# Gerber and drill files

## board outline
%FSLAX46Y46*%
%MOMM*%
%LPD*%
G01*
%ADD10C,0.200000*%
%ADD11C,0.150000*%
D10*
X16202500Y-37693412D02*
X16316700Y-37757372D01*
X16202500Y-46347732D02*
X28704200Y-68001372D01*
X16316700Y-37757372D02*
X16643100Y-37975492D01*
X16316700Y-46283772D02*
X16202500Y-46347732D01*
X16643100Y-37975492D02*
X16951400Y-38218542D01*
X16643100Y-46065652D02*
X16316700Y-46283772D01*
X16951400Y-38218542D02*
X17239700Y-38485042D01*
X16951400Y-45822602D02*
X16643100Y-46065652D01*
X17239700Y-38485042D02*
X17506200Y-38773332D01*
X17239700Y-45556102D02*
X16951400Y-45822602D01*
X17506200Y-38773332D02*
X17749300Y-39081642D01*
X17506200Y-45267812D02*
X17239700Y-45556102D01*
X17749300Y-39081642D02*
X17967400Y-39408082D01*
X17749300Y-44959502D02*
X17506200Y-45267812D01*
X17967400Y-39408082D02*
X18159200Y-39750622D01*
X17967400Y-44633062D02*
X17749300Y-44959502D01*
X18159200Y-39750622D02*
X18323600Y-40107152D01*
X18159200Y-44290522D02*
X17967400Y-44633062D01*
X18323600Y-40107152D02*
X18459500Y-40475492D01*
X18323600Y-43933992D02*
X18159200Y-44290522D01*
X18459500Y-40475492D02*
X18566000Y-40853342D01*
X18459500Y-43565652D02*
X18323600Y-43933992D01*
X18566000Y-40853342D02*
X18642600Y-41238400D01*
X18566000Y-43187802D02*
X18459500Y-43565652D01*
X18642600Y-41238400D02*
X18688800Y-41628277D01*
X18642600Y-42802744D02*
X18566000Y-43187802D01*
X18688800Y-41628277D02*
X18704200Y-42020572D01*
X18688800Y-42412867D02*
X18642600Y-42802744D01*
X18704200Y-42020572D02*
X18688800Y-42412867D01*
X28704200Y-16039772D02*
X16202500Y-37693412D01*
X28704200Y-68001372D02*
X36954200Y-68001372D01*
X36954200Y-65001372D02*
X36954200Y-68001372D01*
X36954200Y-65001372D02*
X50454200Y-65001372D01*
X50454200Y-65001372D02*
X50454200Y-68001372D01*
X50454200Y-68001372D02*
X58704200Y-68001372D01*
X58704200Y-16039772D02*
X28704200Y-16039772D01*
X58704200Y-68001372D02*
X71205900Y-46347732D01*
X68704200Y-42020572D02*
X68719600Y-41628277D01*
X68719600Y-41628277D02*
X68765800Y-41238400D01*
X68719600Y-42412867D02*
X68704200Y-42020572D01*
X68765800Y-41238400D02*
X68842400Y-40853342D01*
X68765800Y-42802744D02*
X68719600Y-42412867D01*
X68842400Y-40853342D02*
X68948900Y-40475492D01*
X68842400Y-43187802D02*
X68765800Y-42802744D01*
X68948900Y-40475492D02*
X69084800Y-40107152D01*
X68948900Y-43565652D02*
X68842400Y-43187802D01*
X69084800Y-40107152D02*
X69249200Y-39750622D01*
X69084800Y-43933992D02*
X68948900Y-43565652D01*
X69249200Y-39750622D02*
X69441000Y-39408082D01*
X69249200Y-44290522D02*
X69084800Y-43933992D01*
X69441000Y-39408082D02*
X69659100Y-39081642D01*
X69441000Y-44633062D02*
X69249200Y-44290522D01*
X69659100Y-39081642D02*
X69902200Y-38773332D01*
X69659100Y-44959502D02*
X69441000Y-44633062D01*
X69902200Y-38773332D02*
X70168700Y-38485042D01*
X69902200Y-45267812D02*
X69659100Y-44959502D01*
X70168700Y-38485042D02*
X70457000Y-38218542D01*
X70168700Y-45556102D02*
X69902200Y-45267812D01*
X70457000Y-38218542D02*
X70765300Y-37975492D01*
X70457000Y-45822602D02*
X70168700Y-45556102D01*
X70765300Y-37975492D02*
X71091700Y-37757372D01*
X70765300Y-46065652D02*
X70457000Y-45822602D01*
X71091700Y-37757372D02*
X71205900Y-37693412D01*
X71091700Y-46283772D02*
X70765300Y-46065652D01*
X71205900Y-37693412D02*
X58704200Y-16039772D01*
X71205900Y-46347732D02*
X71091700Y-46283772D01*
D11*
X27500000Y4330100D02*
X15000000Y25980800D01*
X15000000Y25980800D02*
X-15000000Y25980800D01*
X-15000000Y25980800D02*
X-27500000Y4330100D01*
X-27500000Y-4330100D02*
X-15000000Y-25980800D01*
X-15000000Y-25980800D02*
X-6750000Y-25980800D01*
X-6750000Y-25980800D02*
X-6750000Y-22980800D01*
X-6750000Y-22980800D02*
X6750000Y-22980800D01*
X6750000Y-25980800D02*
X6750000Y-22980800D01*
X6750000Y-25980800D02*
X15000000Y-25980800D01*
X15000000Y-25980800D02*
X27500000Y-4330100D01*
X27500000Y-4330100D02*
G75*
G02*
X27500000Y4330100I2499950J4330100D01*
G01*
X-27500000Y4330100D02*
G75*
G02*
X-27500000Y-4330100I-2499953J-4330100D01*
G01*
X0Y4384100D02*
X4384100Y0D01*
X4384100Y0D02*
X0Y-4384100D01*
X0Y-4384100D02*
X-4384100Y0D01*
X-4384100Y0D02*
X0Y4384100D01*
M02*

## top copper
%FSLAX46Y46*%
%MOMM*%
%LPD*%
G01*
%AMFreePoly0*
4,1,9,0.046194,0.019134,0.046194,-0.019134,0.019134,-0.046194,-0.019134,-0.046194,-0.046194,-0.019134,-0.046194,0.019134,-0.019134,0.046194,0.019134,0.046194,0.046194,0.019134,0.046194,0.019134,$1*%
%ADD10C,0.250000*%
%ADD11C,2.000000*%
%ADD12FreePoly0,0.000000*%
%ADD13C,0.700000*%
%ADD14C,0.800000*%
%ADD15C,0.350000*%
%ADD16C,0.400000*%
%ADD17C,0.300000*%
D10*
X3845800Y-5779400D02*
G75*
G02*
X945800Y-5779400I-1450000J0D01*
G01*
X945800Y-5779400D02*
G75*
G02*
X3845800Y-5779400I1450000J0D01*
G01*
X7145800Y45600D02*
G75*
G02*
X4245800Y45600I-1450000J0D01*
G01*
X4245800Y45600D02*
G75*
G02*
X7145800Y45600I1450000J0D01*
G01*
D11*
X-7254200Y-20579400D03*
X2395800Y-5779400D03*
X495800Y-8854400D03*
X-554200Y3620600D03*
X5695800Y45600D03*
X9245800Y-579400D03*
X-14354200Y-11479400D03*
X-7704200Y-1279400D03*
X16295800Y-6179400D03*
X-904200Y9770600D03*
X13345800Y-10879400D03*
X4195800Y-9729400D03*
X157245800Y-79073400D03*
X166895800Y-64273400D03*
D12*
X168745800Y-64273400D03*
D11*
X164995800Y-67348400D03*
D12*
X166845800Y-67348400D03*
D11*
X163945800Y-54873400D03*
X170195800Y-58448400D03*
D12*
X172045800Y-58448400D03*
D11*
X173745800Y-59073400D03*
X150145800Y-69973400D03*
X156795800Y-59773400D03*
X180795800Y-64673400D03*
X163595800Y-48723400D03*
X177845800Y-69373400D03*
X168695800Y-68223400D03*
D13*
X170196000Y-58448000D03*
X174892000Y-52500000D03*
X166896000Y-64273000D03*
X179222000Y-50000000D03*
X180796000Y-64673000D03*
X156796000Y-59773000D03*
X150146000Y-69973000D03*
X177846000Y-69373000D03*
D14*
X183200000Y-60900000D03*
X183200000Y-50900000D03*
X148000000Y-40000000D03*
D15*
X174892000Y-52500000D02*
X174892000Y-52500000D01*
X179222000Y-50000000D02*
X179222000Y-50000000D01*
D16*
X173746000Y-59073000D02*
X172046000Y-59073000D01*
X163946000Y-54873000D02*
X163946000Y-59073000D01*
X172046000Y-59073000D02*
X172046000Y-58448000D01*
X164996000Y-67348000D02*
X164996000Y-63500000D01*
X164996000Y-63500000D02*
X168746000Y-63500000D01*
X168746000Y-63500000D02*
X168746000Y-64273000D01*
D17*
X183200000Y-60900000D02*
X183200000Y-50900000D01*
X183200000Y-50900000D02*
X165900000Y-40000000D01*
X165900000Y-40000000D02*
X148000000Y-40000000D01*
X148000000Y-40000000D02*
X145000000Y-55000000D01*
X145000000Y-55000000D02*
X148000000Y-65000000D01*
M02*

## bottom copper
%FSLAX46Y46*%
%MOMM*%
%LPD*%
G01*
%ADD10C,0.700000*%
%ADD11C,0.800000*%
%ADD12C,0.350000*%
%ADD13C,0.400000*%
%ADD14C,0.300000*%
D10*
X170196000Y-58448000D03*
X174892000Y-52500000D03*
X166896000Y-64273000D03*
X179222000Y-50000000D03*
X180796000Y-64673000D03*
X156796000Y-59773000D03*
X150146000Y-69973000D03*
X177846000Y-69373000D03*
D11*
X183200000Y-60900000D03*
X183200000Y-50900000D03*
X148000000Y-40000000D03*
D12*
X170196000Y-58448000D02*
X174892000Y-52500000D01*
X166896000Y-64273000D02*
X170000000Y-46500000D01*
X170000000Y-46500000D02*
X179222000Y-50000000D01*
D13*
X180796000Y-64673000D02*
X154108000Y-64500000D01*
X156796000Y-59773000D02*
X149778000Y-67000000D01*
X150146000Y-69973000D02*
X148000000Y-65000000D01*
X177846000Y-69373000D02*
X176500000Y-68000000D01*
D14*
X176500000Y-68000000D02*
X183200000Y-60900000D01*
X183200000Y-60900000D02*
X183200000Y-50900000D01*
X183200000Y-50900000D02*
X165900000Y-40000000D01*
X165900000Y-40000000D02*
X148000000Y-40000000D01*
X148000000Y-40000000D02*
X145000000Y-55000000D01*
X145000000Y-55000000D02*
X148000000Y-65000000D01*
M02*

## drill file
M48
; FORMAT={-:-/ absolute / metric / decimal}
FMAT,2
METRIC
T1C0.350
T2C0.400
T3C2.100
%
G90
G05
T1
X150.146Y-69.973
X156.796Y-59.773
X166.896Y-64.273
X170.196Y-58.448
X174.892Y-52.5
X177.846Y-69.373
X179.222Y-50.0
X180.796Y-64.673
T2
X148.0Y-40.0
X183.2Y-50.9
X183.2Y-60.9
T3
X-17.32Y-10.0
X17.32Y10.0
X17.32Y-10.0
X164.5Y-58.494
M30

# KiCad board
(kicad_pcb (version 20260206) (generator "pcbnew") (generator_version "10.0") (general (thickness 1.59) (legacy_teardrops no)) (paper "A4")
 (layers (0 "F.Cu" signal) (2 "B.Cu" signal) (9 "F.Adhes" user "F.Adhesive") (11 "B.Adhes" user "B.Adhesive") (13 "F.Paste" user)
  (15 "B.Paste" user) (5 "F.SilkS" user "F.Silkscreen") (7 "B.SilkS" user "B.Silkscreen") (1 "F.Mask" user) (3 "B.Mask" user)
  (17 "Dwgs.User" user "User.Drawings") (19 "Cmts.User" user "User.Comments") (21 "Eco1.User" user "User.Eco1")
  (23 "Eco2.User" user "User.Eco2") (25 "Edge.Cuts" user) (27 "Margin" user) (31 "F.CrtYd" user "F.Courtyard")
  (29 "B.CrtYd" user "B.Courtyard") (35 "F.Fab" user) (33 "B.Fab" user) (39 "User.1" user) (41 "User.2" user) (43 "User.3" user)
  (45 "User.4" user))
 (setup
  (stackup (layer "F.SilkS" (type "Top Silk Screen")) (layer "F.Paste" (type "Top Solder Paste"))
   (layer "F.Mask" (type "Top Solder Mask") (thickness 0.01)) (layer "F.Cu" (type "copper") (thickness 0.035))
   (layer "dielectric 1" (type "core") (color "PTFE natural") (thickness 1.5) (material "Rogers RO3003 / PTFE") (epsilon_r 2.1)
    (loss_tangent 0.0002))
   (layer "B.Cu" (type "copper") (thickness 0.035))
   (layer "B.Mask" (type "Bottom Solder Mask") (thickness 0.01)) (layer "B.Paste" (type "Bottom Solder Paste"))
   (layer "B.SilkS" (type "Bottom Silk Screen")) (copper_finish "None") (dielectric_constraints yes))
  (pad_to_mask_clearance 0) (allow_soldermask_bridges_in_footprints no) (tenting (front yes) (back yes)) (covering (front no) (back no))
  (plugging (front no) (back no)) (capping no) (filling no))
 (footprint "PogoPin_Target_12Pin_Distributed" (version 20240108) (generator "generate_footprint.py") (layer "F.Cu")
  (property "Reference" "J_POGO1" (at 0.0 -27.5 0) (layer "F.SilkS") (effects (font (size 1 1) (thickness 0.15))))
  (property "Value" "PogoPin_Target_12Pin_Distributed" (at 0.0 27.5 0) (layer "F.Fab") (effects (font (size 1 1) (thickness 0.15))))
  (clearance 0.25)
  (fp_line (start 27.5 -4.3301) (end 15.0 -25.9808) (stroke (width 0.15) (type solid)) (layer "Edge.Cuts"))
  (fp_line (start 15.0 -25.9808) (end -15.0 -25.9808) (stroke (width 0.15) (type solid)) (layer "Edge.Cuts"))
  (fp_line (start -15.0 -25.9808) (end -27.5 -4.3301) (stroke (width 0.15) (type solid)) (layer "Edge.Cuts"))
  (fp_line (start -27.5 4.3301) (end -15.0 25.9808) (stroke (width 0.15) (type solid)) (layer "Edge.Cuts"))
  (fp_line (start -15.0 25.9808) (end -6.75 25.9808) (stroke (width 0.15) (type solid)) (layer "Edge.Cuts"))
  (fp_line (start -6.75 25.9808) (end -6.75 22.9808) (stroke (width 0.15) (type solid)) (layer "Edge.Cuts"))
  (fp_line (start -6.75 22.9808) (end 6.75 22.9808) (stroke (width 0.15) (type solid)) (layer "Edge.Cuts"))
  (fp_line (start 6.75 25.9808) (end 6.75 22.9808) (stroke (width 0.15) (type solid)) (layer "Edge.Cuts"))
  (fp_line (start 6.75 25.9808) (end 15.0 25.9808) (stroke (width 0.15) (type solid)) (layer "Edge.Cuts"))
  (fp_line (start 15.0 25.9808) (end 27.5 4.3301) (stroke (width 0.15) (type solid)) (layer "Edge.Cuts"))
  (fp_arc (start 27.5 -4.3301) (mid 25.0 0.0) (end 27.5 4.3301) (stroke (width 0.15) (type solid)) (layer "Edge.Cuts"))
  (fp_arc (start -27.5 -4.3301) (mid -25.0 0.0) (end -27.5 4.3301) (stroke (width 0.15) (type solid)) (layer "Edge.Cuts"))
  (fp_line (start 0.0 -4.3841) (end 4.3841 0.0) (stroke (width 0.15) (type solid)) (layer "Edge.Cuts"))
  (fp_line (start 4.3841 0.0) (end 0.0 4.3841) (stroke (width 0.15) (type solid)) (layer "Edge.Cuts"))
  (fp_line (start 0.0 4.3841) (end -4.3841 0.0) (stroke (width 0.15) (type solid)) (layer "Edge.Cuts"))
  (fp_line (start -4.3841 0.0) (end 0.0 -4.3841) (stroke (width 0.15) (type solid)) (layer "Edge.Cuts"))
  (pad "H1" np_thru_hole circle (at 164.5 58.494) (size 2.1 2.1) (drill 2.1) (layers "*.Cu" "*.Mask"))
  (pad "H2" np_thru_hole circle (at 17.3205 10.0) (size 2.1 2.1) (drill 2.1) (layers "*.Cu" "*.Mask"))
  (pad "H3" np_thru_hole circle (at -17.3205 10.0) (size 2.1 2.1) (drill 2.1) (layers "*.Cu" "*.Mask"))
  (pad "H4" np_thru_hole circle (at 17.3205 -10.0) (size 2.1 2.1) (drill 2.1) (layers "*.Cu" "*.Mask"))
  (pad "1" smd circle (at -7.2542 20.5794) (size 2.0 2.0) (layers "F.Cu" "F.Mask") (clearance 0.4) (solder_mask_margin 0.05))
  (pad "2" smd circle (at 2.3958 5.7794) (size 2.0 2.0) (layers "F.Cu" "F.Mask") (clearance 0.4) (solder_mask_margin 0.1))
  (pad "3" smd circle (at 0.4958 8.8544) (size 2.0 2.0) (layers "F.Cu" "F.Mask") (clearance 0.4) (solder_mask_margin 0.1))
  (pad "4" smd circle (at -0.5542 -3.6206) (size 2.0 2.0) (layers "F.Cu" "F.Mask") (clearance 0.4) (solder_mask_margin 0.05))
  (pad "5" smd circle (at 5.6958 -0.0456) (size 2.0 2.0) (layers "F.Cu" "F.Mask") (clearance 0.4) (solder_mask_margin 0.1))
  (pad "6" smd circle (at 9.2458 0.5794) (size 2.0 2.0) (layers "F.Cu" "F.Mask") (clearance 0.4) (solder_mask_margin 0.05))
  (pad "7" smd circle (at -14.3542 11.4794) (size 2.0 2.0) (layers "F.Cu" "F.Mask") (clearance 0.4) (solder_mask_margin 0.05))
  (pad "8" smd circle (at -7.7042 1.2794) (size 2.0 2.0) (layers "F.Cu" "F.Mask") (clearance 0.4) (solder_mask_margin 0.05))
  (pad "9" smd circle (at 16.2958 6.1794) (size 2.0 2.0) (layers "F.Cu" "F.Mask") (clearance 0.4) (solder_mask_margin 0.05))
  (pad "10" smd circle (at -0.9042 -9.7706) (size 2.0 2.0) (layers "F.Cu" "F.Mask") (clearance 0.4) (solder_mask_margin 0.05))
  (pad "11" smd circle (at 13.3458 10.8794) (size 2.0 2.0) (layers "F.Cu" "F.Mask") (clearance 0.4) (solder_mask_margin 0.05))
  (pad "12" smd circle (at 4.1958 9.7294) (size 2.0 2.0) (layers "F.Cu" "F.Mask") (clearance 0.4) (solder_mask_margin 0.05))
  (fp_circle (center 2.3958 5.7794) (end 3.8458 5.7794) (stroke (width 0.25) (type solid)) (fill none) (layer "F.Cu"))
  (fp_circle (center 5.6958 -0.0456) (end 7.1458 -0.0456) (stroke (width 0.25) (type solid)) (fill none) (layer "F.Cu")))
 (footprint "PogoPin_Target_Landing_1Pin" (at 157.2458 79.0734) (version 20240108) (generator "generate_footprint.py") (layer "F.Cu")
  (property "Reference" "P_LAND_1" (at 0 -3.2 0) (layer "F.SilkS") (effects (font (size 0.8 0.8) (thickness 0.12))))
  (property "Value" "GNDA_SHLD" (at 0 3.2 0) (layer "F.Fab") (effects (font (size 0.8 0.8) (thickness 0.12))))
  (pad "1" smd circle (at 0 0) (size 2.0 2.0) (layers "F.Cu" "F.Mask") (clearance 0.4) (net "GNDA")))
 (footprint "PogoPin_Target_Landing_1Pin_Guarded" (at 166.8958 64.2734) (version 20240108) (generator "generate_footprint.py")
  (layer "F.Cu")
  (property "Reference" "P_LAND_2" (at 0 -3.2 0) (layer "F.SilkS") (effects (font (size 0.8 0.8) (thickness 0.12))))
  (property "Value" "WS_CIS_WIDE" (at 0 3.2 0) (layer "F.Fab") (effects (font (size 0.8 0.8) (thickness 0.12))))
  (pad "1" smd circle (at 0 0) (size 2.0 2.0) (layers "F.Cu" "F.Mask") (clearance 0.4) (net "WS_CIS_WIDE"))
  (pad "2" smd custom (at 1.85 0) (size 0.1 0.1) (layers "F.Cu") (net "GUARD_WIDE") (clearance 0.3)
   (options (clearance outline) (anchor circle)) (primitives)))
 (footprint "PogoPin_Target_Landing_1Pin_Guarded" (at 164.9958 67.3484) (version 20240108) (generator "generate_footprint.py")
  (layer "F.Cu")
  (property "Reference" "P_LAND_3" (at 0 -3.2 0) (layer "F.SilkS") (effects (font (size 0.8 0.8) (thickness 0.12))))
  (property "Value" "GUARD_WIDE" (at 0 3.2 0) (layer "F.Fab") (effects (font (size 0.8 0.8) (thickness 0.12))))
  (pad "1" smd circle (at 0 0) (size 2.0 2.0) (layers "F.Cu" "F.Mask") (clearance 0.4) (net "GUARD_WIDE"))
  (pad "2" smd custom (at 1.85 0) (size 0.1 0.1) (layers "F.Cu") (clearance 0.3) (options (clearance outline) (anchor circle)) (primitives)))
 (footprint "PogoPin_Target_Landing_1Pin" (at 163.9458 54.8734) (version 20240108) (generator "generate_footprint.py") (layer "F.Cu")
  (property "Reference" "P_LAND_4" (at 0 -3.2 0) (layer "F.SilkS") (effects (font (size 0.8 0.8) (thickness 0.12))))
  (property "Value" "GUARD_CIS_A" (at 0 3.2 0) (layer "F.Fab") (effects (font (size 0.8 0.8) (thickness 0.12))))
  (pad "1" smd circle (at 0 0) (size 2.0 2.0) (layers "F.Cu" "F.Mask") (clearance 0.4) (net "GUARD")))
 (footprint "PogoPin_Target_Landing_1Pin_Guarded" (at 170.1958 58.4484) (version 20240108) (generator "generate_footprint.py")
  (layer "F.Cu")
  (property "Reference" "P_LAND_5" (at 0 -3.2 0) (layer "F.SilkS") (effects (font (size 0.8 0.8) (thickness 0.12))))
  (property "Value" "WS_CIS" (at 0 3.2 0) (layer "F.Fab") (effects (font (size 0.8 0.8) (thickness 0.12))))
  (pad "1" smd circle (at 0 0) (size 2.0 2.0) (layers "F.Cu" "F.Mask") (clearance 0.4) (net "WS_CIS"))
  (pad "2" smd custom (at 1.85 0) (size 0.1 0.1) (layers "F.Cu") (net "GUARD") (clearance 0.3) (options (clearance outline) (anchor circle))
   (primitives)))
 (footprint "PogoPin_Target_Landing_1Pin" (at 173.7458 59.0734) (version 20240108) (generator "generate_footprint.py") (layer "F.Cu")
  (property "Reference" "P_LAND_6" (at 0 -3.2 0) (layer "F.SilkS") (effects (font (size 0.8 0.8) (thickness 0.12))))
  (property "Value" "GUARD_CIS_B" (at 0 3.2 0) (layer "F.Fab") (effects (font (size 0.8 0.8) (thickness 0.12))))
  (pad "1" smd circle (at 0 0) (size 2.0 2.0) (layers "F.Cu" "F.Mask") (clearance 0.4) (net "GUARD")))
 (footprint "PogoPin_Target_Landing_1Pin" (at 150.1458 69.9734) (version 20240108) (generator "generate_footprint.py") (layer "F.Cu")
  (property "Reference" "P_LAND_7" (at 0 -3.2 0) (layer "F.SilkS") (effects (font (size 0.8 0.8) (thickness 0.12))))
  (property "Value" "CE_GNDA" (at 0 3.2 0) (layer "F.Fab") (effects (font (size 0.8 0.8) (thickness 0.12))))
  (pad "1" smd circle (at 0 0) (size 2.0 2.0) (layers "F.Cu" "F.Mask") (clearance 0.4) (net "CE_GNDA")))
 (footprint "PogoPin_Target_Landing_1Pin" (at 156.7958 59.7734) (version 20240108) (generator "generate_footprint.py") (layer "F.Cu")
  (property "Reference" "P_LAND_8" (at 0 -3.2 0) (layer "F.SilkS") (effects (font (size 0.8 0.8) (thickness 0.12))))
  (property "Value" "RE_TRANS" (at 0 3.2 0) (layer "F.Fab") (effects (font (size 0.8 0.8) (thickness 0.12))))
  (pad "1" smd circle (at 0 0) (size 2.0 2.0) (layers "F.Cu" "F.Mask") (clearance 0.4) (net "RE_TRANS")))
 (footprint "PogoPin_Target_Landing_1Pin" (at 180.7958 64.6734) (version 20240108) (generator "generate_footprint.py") (layer "F.Cu")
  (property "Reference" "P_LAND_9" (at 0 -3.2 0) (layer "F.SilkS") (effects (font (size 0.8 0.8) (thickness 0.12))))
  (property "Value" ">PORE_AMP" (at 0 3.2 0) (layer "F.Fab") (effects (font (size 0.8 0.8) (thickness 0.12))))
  (pad "1" smd circle (at 0 0) (size 2.0 2.0) (layers "F.Cu" "F.Mask") (clearance 0.4) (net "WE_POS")))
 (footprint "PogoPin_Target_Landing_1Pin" (at 163.5958 48.7234) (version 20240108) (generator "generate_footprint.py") (layer "F.Cu")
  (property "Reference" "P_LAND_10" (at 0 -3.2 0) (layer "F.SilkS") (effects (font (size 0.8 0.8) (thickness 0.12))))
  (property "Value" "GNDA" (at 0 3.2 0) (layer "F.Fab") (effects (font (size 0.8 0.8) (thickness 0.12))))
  (pad "1" smd circle (at 0 0) (size 2.0 2.0) (layers "F.Cu" "F.Mask") (clearance 0.4) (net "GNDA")))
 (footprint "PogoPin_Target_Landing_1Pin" (at 177.8458 69.3734) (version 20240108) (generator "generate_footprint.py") (layer "F.Cu")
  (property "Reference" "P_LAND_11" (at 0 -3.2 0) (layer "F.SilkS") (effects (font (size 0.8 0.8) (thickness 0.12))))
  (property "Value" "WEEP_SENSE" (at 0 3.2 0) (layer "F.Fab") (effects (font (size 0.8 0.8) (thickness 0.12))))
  (pad "1" smd circle (at 0 0) (size 2.0 2.0) (layers "F.Cu" "F.Mask") (clearance 0.4) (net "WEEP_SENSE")))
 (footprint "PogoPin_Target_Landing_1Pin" (at 168.6958 68.2234) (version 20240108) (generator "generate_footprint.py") (layer "F.Cu")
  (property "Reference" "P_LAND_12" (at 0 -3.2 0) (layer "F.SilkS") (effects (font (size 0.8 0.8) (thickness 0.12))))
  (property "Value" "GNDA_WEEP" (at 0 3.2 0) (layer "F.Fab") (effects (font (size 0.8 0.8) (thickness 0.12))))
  (pad "1" smd circle (at 0 0) (size 2.0 2.0) (layers "F.Cu" "F.Mask") (clearance 0.4) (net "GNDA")))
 (gr_line (start 16.2025 37.693412) (end 16.3167 37.757372) (stroke (width 0.2) (type default)) (layer "Edge.Cuts"))
 (gr_line (start 16.2025 46.347732) (end 28.7042 68.001372) (stroke (width 0.2) (type default)) (layer "Edge.Cuts"))
 (gr_line (start 16.3167 37.757372) (end 16.6431 37.975492) (stroke (width 0.2) (type default)) (layer "Edge.Cuts"))
 (gr_line (start 16.3167 46.283772) (end 16.2025 46.347732) (stroke (width 0.2) (type default)) (layer "Edge.Cuts"))
 (gr_line (start 16.6431 37.975492) (end 16.9514 38.218542) (stroke (width 0.2) (type default)) (layer "Edge.Cuts"))
 (gr_line (start 16.6431 46.065652) (end 16.3167 46.283772) (stroke (width 0.2) (type default)) (layer "Edge.Cuts"))
 (gr_line (start 16.9514 38.218542) (end 17.2397 38.485042) (stroke (width 0.2) (type default)) (layer "Edge.Cuts"))
 (gr_line (start 16.9514 45.822602) (end 16.6431 46.065652) (stroke (width 0.2) (type default)) (layer "Edge.Cuts"))
 (gr_line (start 17.2397 38.485042) (end 17.5062 38.773332) (stroke (width 0.2) (type default)) (layer "Edge.Cuts"))
 (gr_line (start 17.2397 45.556102) (end 16.9514 45.822602) (stroke (width 0.2) (type default)) (layer "Edge.Cuts"))
 (gr_line (start 17.5062 38.773332) (end 17.7493 39.081642) (stroke (width 0.2) (type default)) (layer "Edge.Cuts"))
 (gr_line (start 17.5062 45.267812) (end 17.2397 45.556102) (stroke (width 0.2) (type default)) (layer "Edge.Cuts"))
 (gr_line (start 17.7493 39.081642) (end 17.9674 39.408082) (stroke (width 0.2) (type default)) (layer "Edge.Cuts"))
 (gr_line (start 17.7493 44.959502) (end 17.5062 45.267812) (stroke (width 0.2) (type default)) (layer "Edge.Cuts"))
 (gr_line (start 17.9674 39.408082) (end 18.1592 39.750622) (stroke (width 0.2) (type default)) (layer "Edge.Cuts"))
 (gr_line (start 17.9674 44.633062) (end 17.7493 44.959502) (stroke (width 0.2) (type default)) (layer "Edge.Cuts"))
 (gr_line (start 18.1592 39.750622) (end 18.3236 40.107152) (stroke (width 0.2) (type default)) (layer "Edge.Cuts"))
 (gr_line (start 18.1592 44.290522) (end 17.9674 44.633062) (stroke (width 0.2) (type default)) (layer "Edge.Cuts"))
 (gr_line (start 18.3236 40.107152) (end 18.4595 40.475492) (stroke (width 0.2) (type default)) (layer "Edge.Cuts"))
 (gr_line (start 18.3236 43.933992) (end 18.1592 44.290522) (stroke (width 0.2) (type default)) (layer "Edge.Cuts"))
 (gr_line (start 18.4595 40.475492) (end 18.566 40.853342) (stroke (width 0.2) (type default)) (layer "Edge.Cuts"))
 (gr_line (start 18.4595 43.565652) (end 18.3236 43.933992) (stroke (width 0.2) (type default)) (layer "Edge.Cuts"))
 (gr_line (start 18.566 40.853342) (end 18.6426 41.2384) (stroke (width 0.2) (type default)) (layer "Edge.Cuts"))
 (gr_line (start 18.566 43.187802) (end 18.4595 43.565652) (stroke (width 0.2) (type default)) (layer "Edge.Cuts"))
 (gr_line (start 18.6426 41.2384) (end 18.6888 41.628277) (stroke (width 0.2) (type default)) (layer "Edge.Cuts"))
 (gr_line (start 18.6426 42.802744) (end 18.566 43.187802) (stroke (width 0.2) (type default)) (layer "Edge.Cuts"))
 (gr_line (start 18.6888 41.628277) (end 18.7042 42.020572) (stroke (width 0.2) (type default)) (layer "Edge.Cuts"))
 (gr_line (start 18.6888 42.412867) (end 18.6426 42.802744) (stroke (width 0.2) (type default)) (layer "Edge.Cuts"))
 (gr_line (start 18.7042 42.020572) (end 18.6888 42.412867) (stroke (width 0.2) (type default)) (layer "Edge.Cuts"))
 (gr_line (start 28.7042 16.039772) (end 16.2025 37.693412) (stroke (width 0.2) (type default)) (layer "Edge.Cuts"))
 (gr_line (start 28.7042 68.001372) (end 36.9542 68.001372) (stroke (width 0.2) (type default)) (layer "Edge.Cuts"))
 (gr_line (start 36.9542 65.001372) (end 36.9542 68.001372) (stroke (width 0.2) (type default)) (layer "Edge.Cuts"))
 (gr_line (start 36.9542 65.001372) (end 50.4542 65.001372) (stroke (width 0.2) (type default)) (layer "Edge.Cuts"))
 (gr_line (start 50.4542 65.001372) (end 50.4542 68.001372) (stroke (width 0.2) (type default)) (layer "Edge.Cuts"))
 (gr_line (start 50.4542 68.001372) (end 58.7042 68.001372) (stroke (width 0.2) (type default)) (layer "Edge.Cuts"))
 (gr_line (start 58.7042 16.039772) (end 28.7042 16.039772) (stroke (width 0.2) (type default)) (layer "Edge.Cuts"))
 (gr_line (start 58.7042 68.001372) (end 71.2059 46.347732) (stroke (width 0.2) (type default)) (layer "Edge.Cuts"))
 (gr_line (start 68.7042 42.020572) (end 68.7196 41.628277) (stroke (width 0.2) (type default)) (layer "Edge.Cuts"))
 (gr_line (start 68.7196 41.628277) (end 68.7658 41.2384) (stroke (width 0.2) (type default)) (layer "Edge.Cuts"))
 (gr_line (start 68.7196 42.412867) (end 68.7042 42.020572) (stroke (width 0.2) (type default)) (layer "Edge.Cuts"))
 (gr_line (start 68.7658 41.2384) (end 68.8424 40.853342) (stroke (width 0.2) (type default)) (layer "Edge.Cuts"))
 (gr_line (start 68.7658 42.802744) (end 68.7196 42.412867) (stroke (width 0.2) (type default)) (layer "Edge.Cuts"))
 (gr_line (start 68.8424 40.853342) (end 68.9489 40.475492) (stroke (width 0.2) (type default)) (layer "Edge.Cuts"))
 (gr_line (start 68.8424 43.187802) (end 68.7658 42.802744) (stroke (width 0.2) (type default)) (layer "Edge.Cuts"))
 (gr_line (start 68.9489 40.475492) (end 69.0848 40.107152) (stroke (width 0.2) (type default)) (layer "Edge.Cuts"))
 (gr_line (start 68.9489 43.565652) (end 68.8424 43.187802) (stroke (width 0.2) (type default)) (layer "Edge.Cuts"))
 (gr_line (start 69.0848 40.107152) (end 69.2492 39.750622) (stroke (width 0.2) (type default)) (layer "Edge.Cuts"))
 (gr_line (start 69.0848 43.933992) (end 68.9489 43.565652) (stroke (width 0.2) (type default)) (layer "Edge.Cuts"))
 (gr_line (start 69.2492 39.750622) (end 69.441 39.408082) (stroke (width 0.2) (type default)) (layer "Edge.Cuts"))
 (gr_line (start 69.2492 44.290522) (end 69.0848 43.933992) (stroke (width 0.2) (type default)) (layer "Edge.Cuts"))
 (gr_line (start 69.441 39.408082) (end 69.6591 39.081642) (stroke (width 0.2) (type default)) (layer "Edge.Cuts"))
 (gr_line (start 69.441 44.633062) (end 69.2492 44.290522) (stroke (width 0.2) (type default)) (layer "Edge.Cuts"))
 (gr_line (start 69.6591 39.081642) (end 69.9022 38.773332) (stroke (width 0.2) (type default)) (layer "Edge.Cuts"))
 (gr_line (start 69.6591 44.959502) (end 69.441 44.633062) (stroke (width 0.2) (type default)) (layer "Edge.Cuts"))
 (gr_line (start 69.9022 38.773332) (end 70.1687 38.485042) (stroke (width 0.2) (type default)) (layer "Edge.Cuts"))
 (gr_line (start 69.9022 45.267812) (end 69.6591 44.959502) (stroke (width 0.2) (type default)) (layer "Edge.Cuts"))
 (gr_line (start 70.1687 38.485042) (end 70.457 38.218542) (stroke (width 0.2) (type default)) (layer "Edge.Cuts"))
 (gr_line (start 70.1687 45.556102) (end 69.9022 45.267812) (stroke (width 0.2) (type default)) (layer "Edge.Cuts"))
 (gr_line (start 70.457 38.218542) (end 70.7653 37.975492) (stroke (width 0.2) (type default)) (layer "Edge.Cuts"))
 (gr_line (start 70.457 45.822602) (end 70.1687 45.556102) (stroke (width 0.2) (type default)) (layer "Edge.Cuts"))
 (gr_line (start 70.7653 37.975492) (end 71.0917 37.757372) (stroke (width 0.2) (type default)) (layer "Edge.Cuts"))
 (gr_line (start 70.7653 46.065652) (end 70.457 45.822602) (stroke (width 0.2) (type default)) (layer "Edge.Cuts"))
 (gr_line (start 71.0917 37.757372) (end 71.2059 37.693412) (stroke (width 0.2) (type default)) (layer "Edge.Cuts"))
 (gr_line (start 71.0917 46.283772) (end 70.7653 46.065652) (stroke (width 0.2) (type default)) (layer "Edge.Cuts"))
 (gr_line (start 71.2059 37.693412) (end 58.7042 16.039772) (stroke (width 0.2) (type default)) (layer "Edge.Cuts"))
 (gr_line (start 71.2059 46.347732) (end 71.0917 46.283772) (stroke (width 0.2) (type default)) (layer "Edge.Cuts"))
 (segment (start 170.1960 58.4480) (end 174.8920 52.5000) (width 0.35) (layer "B.Cu") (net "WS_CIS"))
 (segment (start 174.8920 52.5000) (end 174.8920 52.5000) (width 0.35) (layer "F.Cu") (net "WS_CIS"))
 (via (at 170.1960 58.4480) (size 0.7) (drill 0.35) (layers "F.Cu" "B.Cu") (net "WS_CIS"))
 (via (at 174.8920 52.5000) (size 0.7) (drill 0.35) (layers "F.Cu" "B.Cu") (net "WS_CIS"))
 (segment (start 166.8960 64.2730) (end 170.0000 46.5000) (width 0.35) (layer "B.Cu") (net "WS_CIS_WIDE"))
 (segment (start 170.0000 46.5000) (end 179.2220 50.0000) (width 0.35) (layer "B.Cu") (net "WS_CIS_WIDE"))
 (segment (start 179.2220 50.0000) (end 179.2220 50.0000) (width 0.35) (layer "F.Cu") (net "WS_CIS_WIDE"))
 (via (at 166.8960 64.2730) (size 0.7) (drill 0.35) (layers "F.Cu" "B.Cu") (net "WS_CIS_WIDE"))
 (via (at 179.2220 50.0000) (size 0.7) (drill 0.35) (layers "F.Cu" "B.Cu") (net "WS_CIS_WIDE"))
 (segment (start 173.7460 59.0730) (end 172.0460 59.0730) (width 0.4) (layer "F.Cu") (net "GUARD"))
 (segment (start 163.9460 54.8730) (end 163.9460 59.0730) (width 0.4) (layer "F.Cu") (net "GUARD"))
 (segment (start 172.0460 59.0730) (end 172.0460 58.4480) (width 0.4) (layer "F.Cu") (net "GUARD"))
 (segment (start 164.9960 67.3480) (end 164.9960 63.5000) (width 0.4) (layer "F.Cu") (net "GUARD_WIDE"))
 (segment (start 164.9960 63.5000) (end 168.7460 63.5000) (width 0.4) (layer "F.Cu") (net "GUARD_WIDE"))
 (segment (start 168.7460 63.5000) (end 168.7460 64.2730) (width 0.4) (layer "F.Cu") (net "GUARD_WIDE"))
 (segment (start 180.7960 64.6730) (end 154.1080 64.5000) (width 0.4) (layer "B.Cu") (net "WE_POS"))
 (via (at 180.7960 64.6730) (size 0.7) (drill 0.35) (layers "F.Cu" "B.Cu") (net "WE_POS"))
 (segment (start 156.7960 59.7730) (end 149.7780 67.0000) (width 0.4) (layer "B.Cu") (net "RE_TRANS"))
 (via (at 156.7960 59.7730) (size 0.7) (drill 0.35) (layers "F.Cu" "B.Cu") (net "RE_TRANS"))
 (segment (start 150.1460 69.9730) (end 148.0000 65.0000) (width 0.4) (layer "B.Cu") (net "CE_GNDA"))
 (via (at 150.1460 69.9730) (size 0.7) (drill 0.35) (layers "F.Cu" "B.Cu") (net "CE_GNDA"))
 (via (at 177.8460 69.3730) (size 0.7) (drill 0.35) (layers "F.Cu" "B.Cu") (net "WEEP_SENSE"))
 (segment (start 177.8460 69.3730) (end 176.5000 68.0000) (width 0.4) (layer "B.Cu") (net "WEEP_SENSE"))
 (segment (start 176.5000 68.0000) (end 183.2000 60.9000) (width 0.3) (layer "B.Cu") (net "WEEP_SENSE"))
 (segment (start 183.2000 60.9000) (end 183.2000 50.9000) (width 0.3) (layer "B.Cu") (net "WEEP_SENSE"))
 (segment (start 183.2000 50.9000) (end 165.9000 40.0000) (width 0.3) (layer "B.Cu") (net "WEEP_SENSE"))
 (segment (start 165.9000 40.0000) (end 148.0000 40.0000) (width 0.3) (layer "B.Cu") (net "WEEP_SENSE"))
 (segment (start 148.0000 40.0000) (end 145.0000 55.0000) (width 0.3) (layer "B.Cu") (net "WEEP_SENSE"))
 (segment (start 145.0000 55.0000) (end 148.0000 65.0000) (width 0.3) (layer "B.Cu") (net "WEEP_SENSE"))
 (segment (start 183.2000 60.9000) (end 183.2000 50.9000) (width 0.3) (layer "F.Cu") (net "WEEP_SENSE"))
 (segment (start 183.2000 50.9000) (end 165.9000 40.0000) (width 0.3) (layer "F.Cu") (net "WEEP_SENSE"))
 (segment (start 165.9000 40.0000) (end 148.0000 40.0000) (width 0.3) (layer "F.Cu") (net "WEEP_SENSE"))
 (segment (start 148.0000 40.0000) (end 145.0000 55.0000) (width 0.3) (layer "F.Cu") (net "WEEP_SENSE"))
 (segment (start 145.0000 55.0000) (end 148.0000 65.0000) (width 0.3) (layer "F.Cu") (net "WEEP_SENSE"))
 (via (at 183.2000 60.9000) (size 0.8) (drill 0.4) (layers "F.Cu" "B.Cu") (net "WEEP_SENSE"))
 (via (at 183.2000 50.9000) (size 0.8) (drill 0.4) (layers "F.Cu" "B.Cu") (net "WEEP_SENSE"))
 (via (at 148.0000 40.0000) (size 0.8) (drill 0.4) (layers "F.Cu" "B.Cu") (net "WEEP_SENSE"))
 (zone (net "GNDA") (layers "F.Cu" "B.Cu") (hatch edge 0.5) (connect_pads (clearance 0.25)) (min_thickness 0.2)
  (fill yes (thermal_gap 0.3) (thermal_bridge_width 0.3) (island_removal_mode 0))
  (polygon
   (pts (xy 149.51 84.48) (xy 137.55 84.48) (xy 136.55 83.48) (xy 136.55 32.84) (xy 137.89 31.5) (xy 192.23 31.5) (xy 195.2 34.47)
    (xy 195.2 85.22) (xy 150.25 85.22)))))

